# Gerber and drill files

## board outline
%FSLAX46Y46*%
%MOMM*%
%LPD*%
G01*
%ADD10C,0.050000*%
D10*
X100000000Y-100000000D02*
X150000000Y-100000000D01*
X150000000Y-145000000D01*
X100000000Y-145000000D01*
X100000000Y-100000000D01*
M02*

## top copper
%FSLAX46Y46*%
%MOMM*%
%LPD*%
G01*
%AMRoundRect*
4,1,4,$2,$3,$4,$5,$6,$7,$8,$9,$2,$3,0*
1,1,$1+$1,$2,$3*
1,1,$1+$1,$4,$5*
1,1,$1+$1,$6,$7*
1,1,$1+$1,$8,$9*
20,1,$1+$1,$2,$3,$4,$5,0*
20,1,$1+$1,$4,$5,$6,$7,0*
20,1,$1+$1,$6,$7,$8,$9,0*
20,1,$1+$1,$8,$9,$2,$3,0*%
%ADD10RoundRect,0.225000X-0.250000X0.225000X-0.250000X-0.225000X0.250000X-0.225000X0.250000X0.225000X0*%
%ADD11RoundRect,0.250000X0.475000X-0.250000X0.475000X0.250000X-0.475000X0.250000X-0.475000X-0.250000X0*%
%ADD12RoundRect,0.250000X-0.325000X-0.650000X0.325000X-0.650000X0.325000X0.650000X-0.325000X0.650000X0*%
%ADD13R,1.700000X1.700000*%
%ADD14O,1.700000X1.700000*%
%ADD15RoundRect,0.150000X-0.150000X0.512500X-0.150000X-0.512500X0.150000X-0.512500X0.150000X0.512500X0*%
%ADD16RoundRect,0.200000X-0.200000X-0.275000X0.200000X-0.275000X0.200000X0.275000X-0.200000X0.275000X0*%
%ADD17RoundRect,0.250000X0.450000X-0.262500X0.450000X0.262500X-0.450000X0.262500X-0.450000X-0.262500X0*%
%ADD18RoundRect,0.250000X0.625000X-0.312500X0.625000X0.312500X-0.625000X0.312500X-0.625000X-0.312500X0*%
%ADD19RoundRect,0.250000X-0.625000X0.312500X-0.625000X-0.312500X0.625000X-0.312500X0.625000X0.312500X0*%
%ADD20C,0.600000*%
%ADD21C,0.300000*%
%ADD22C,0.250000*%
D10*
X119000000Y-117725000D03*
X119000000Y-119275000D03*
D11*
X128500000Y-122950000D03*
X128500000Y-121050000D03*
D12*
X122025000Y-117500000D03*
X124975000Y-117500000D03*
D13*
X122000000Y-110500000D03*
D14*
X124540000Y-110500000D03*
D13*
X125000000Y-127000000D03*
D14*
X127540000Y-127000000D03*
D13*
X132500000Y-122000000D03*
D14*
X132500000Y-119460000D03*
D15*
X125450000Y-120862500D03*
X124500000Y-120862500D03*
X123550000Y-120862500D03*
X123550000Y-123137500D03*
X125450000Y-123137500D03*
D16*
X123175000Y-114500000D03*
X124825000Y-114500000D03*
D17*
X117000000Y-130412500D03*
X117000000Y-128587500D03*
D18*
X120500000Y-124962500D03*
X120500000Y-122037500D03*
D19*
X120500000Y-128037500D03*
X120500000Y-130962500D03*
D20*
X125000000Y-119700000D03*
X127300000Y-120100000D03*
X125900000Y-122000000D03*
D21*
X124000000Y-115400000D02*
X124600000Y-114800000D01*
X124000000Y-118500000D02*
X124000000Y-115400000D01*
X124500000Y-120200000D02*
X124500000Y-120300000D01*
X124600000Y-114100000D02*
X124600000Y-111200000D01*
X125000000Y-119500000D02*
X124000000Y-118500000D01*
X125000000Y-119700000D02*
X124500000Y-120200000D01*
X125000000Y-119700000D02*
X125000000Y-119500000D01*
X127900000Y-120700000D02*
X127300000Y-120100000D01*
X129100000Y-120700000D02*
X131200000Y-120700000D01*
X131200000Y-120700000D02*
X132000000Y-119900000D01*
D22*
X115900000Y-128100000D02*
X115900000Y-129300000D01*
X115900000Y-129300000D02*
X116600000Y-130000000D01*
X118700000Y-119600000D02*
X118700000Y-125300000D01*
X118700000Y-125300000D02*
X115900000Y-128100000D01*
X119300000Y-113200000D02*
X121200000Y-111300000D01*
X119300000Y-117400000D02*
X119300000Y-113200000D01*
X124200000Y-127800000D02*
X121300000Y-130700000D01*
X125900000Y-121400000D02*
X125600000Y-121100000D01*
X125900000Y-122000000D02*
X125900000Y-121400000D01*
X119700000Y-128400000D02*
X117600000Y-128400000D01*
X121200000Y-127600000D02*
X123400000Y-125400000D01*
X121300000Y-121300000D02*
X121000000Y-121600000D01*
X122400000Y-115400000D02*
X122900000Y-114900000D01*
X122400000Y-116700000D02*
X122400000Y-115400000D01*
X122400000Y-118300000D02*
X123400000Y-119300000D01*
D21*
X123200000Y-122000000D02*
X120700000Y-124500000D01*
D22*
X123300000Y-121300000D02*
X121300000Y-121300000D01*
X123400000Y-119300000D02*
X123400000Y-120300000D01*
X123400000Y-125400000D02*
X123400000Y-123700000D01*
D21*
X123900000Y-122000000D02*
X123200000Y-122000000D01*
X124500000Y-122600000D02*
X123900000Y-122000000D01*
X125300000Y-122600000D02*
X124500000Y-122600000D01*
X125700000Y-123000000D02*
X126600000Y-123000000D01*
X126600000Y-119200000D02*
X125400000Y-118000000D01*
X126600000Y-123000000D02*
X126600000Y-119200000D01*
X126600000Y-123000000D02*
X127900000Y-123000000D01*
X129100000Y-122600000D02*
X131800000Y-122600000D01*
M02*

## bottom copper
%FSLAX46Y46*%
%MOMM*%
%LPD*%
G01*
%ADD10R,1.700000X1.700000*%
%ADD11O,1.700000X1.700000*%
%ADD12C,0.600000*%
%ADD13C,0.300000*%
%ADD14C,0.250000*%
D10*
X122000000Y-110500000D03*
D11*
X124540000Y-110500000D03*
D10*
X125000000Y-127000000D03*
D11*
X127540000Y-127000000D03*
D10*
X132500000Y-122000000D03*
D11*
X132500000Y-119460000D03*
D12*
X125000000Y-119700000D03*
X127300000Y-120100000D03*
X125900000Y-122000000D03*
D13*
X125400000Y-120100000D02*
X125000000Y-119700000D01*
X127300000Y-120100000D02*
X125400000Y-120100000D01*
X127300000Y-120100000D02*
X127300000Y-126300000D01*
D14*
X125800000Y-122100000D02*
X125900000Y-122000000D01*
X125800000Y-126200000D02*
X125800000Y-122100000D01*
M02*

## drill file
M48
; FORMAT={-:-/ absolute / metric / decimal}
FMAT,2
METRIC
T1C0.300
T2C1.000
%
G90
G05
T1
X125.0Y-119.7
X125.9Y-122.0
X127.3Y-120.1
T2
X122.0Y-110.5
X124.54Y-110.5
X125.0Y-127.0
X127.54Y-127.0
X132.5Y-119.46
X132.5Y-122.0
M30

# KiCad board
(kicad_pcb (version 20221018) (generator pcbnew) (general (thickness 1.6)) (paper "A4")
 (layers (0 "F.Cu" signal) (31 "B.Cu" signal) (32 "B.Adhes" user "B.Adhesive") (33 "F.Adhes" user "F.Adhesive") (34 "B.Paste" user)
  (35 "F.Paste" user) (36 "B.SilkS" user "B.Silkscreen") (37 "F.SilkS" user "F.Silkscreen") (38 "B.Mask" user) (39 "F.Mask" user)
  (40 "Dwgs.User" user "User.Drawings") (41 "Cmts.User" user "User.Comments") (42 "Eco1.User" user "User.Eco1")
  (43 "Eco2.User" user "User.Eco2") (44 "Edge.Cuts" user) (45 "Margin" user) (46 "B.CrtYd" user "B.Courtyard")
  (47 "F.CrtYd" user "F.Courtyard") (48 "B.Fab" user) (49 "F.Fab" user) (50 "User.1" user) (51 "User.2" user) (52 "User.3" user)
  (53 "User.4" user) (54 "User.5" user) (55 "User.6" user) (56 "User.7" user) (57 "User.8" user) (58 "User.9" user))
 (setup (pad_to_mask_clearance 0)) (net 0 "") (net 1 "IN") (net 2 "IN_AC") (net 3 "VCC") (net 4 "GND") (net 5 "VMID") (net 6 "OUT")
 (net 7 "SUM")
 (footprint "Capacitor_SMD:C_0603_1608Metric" (layer "F.Cu") (at 119 118.5 -90)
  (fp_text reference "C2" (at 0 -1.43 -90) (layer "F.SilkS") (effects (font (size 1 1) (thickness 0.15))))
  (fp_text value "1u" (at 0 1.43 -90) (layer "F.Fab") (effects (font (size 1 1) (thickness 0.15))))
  (pad "1" smd roundrect (at -0.775 0 270) (size 0.9 0.95) (layers "F.Cu" "F.Paste" "F.Mask") (roundrect_rratio 0.25) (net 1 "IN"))
  (pad "2" smd roundrect (at 0.775 0 270) (size 0.9 0.95) (layers "F.Cu" "F.Paste" "F.Mask") (roundrect_rratio 0.25) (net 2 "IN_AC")))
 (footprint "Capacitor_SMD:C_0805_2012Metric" (layer "F.Cu") (at 128.5 122 90)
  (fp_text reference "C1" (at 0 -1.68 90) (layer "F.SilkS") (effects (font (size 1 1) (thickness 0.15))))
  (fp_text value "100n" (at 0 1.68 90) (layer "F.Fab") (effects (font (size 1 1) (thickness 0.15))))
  (pad "1" smd roundrect (at -0.95 0 90) (size 1 1.45) (layers "F.Cu" "F.Paste" "F.Mask") (roundrect_rratio 0.25) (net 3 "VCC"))
  (pad "2" smd roundrect (at 0.95 0 90) (size 1 1.45) (layers "F.Cu" "F.Paste" "F.Mask") (roundrect_rratio 0.25) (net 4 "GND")))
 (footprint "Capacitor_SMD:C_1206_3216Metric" (layer "F.Cu") (at 123.5 117.5)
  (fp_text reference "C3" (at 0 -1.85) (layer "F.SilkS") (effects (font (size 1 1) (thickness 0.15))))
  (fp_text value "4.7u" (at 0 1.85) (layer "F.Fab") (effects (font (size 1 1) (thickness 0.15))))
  (pad "1" smd roundrect (at -1.475 0) (size 1.15 1.8) (layers "F.Cu" "F.Paste" "F.Mask") (roundrect_rratio 0.217391) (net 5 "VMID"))
  (pad "2" smd roundrect (at 1.475 0) (size 1.15 1.8) (layers "F.Cu" "F.Paste" "F.Mask") (roundrect_rratio 0.217391) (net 3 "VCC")))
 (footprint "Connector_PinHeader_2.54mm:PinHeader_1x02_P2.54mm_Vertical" (layer "F.Cu") (at 122 110.5 90)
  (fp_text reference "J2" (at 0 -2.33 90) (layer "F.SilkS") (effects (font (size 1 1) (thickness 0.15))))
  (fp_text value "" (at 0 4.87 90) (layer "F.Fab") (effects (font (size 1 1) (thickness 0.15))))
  (pad "1" thru_hole rect (at 0 0 90) (size 1.7 1.7) (drill 1) (layers "*.Cu" "*.Mask") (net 1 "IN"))
  (pad "2" thru_hole oval (at 0 2.54 90) (size 1.7 1.7) (drill 1) (layers "*.Cu" "*.Mask") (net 4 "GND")))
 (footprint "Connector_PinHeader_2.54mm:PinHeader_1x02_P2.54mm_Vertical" (layer "F.Cu") (at 125 127 90)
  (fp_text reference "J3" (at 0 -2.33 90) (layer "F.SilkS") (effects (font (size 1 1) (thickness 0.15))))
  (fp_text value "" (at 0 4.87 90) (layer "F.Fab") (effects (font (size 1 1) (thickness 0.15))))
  (pad "1" thru_hole rect (at 0 0 90) (size 1.7 1.7) (drill 1) (layers "*.Cu" "*.Mask") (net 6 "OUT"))
  (pad "2" thru_hole oval (at 0 2.54 90) (size 1.7 1.7) (drill 1) (layers "*.Cu" "*.Mask") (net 4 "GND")))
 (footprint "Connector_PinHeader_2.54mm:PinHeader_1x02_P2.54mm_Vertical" (layer "F.Cu") (at 132.5 122 180)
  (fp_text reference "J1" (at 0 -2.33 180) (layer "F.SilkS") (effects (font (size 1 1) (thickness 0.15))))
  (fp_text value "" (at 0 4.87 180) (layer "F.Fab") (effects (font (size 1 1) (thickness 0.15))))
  (pad "1" thru_hole rect (at 0 0 180) (size 1.7 1.7) (drill 1) (layers "*.Cu" "*.Mask") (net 3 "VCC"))
  (pad "2" thru_hole oval (at 0 2.54 180) (size 1.7 1.7) (drill 1) (layers "*.Cu" "*.Mask") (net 4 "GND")))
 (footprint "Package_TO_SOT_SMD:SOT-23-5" (layer "F.Cu") (at 124.5 122 -90)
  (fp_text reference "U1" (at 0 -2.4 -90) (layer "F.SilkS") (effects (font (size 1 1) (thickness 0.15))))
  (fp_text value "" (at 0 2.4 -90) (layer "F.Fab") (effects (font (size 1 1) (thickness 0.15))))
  (pad "1" smd roundrect (at -1.1375 -0.95 270) (size 1.325 0.6) (layers "F.Cu" "F.Paste" "F.Mask") (roundrect_rratio 0.25) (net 6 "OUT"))
  (pad "2" smd roundrect (at -1.1375 0 270) (size 1.325 0.6) (layers "F.Cu" "F.Paste" "F.Mask") (roundrect_rratio 0.25) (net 4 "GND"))
  (pad "3" smd roundrect (at -1.1375 0.95 270) (size 1.325 0.6) (layers "F.Cu" "F.Paste" "F.Mask") (roundrect_rratio 0.25) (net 5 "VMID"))
  (pad "4" smd roundrect (at 1.1375 0.95 270) (size 1.325 0.6) (layers "F.Cu" "F.Paste" "F.Mask") (roundrect_rratio 0.25) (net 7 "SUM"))
  (pad "5" smd roundrect (at 1.1375 -0.95 270) (size 1.325 0.6) (layers "F.Cu" "F.Paste" "F.Mask") (roundrect_rratio 0.25) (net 3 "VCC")))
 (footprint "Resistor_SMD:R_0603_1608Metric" (layer "F.Cu") (at 124 114.5)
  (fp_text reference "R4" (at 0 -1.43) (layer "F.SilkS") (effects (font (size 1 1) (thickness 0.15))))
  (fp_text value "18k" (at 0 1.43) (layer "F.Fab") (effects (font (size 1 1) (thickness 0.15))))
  (pad "1" smd roundrect (at -0.825 0) (size 0.8 0.95) (layers "F.Cu" "F.Paste" "F.Mask") (roundrect_rratio 0.25) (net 5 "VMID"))
  (pad "2" smd roundrect (at 0.825 0) (size 0.8 0.95) (layers "F.Cu" "F.Paste" "F.Mask") (roundrect_rratio 0.25) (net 4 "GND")))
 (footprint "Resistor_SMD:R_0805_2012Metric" (layer "F.Cu") (at 117 129.5 90)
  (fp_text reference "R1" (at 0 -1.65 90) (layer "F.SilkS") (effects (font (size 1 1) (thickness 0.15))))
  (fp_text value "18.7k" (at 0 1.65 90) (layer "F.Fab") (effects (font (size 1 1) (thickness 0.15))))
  (pad "1" smd roundrect (at -0.9125 0 90) (size 1.025 1.4) (layers "F.Cu" "F.Paste" "F.Mask") (roundrect_rratio 0.243902) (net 2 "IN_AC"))
  (pad "2" smd roundrect (at 0.9125 0 90) (size 1.025 1.4) (layers "F.Cu" "F.Paste" "F.Mask") (roundrect_rratio 0.243902) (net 7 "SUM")))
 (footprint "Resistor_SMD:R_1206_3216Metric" (layer "F.Cu") (at 120.5 123.5 90)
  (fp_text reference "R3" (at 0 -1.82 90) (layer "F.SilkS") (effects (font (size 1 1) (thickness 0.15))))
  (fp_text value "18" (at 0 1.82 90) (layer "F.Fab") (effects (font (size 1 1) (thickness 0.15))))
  (pad "1" smd roundrect (at -1.4625 0 90) (size 1.125 1.75) (layers "F.Cu" "F.Paste" "F.Mask") (roundrect_rratio 0.222222) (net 3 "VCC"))
  (pad "2" smd roundrect (at 1.4625 0 90) (size 1.125 1.75) (layers "F.Cu" "F.Paste" "F.Mask") (roundrect_rratio 0.222222) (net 5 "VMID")))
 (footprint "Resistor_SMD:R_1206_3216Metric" (layer "F.Cu") (at 120.5 129.5 -90)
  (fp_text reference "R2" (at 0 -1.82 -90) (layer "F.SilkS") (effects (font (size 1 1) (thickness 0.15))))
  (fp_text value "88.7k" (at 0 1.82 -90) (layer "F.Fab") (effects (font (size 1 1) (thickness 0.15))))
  (pad "1" smd roundrect (at -1.4625 0 270) (size 1.125 1.75) (layers "F.Cu" "F.Paste" "F.Mask") (roundrect_rratio 0.222222) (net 7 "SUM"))
  (pad "2" smd roundrect (at 1.4625 0 270) (size 1.125 1.75) (layers "F.Cu" "F.Paste" "F.Mask") (roundrect_rratio 0.222222) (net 6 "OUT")))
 (gr_rect (start 100 100) (end 150 145) (stroke (width 0.05) (type default)) (fill none) (layer "Edge.Cuts"))
 (segment (start 124 115.4) (end 124.6 114.8) (width 0.3) (layer "F.Cu") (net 4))
 (segment (start 124 118.5) (end 124 115.4) (width 0.3) (layer "F.Cu") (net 4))
 (segment (start 124.5 120.2) (end 124.5 120.3) (width 0.3) (layer "F.Cu") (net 4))
 (segment (start 124.6 114.1) (end 124.6 111.2) (width 0.3) (layer "F.Cu") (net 4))
 (segment (start 125 119.5) (end 124 118.5) (width 0.3) (layer "F.Cu") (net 4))
 (segment (start 125 119.7) (end 124.5 120.2) (width 0.3) (layer "F.Cu") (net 4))
 (segment (start 125 119.7) (end 125 119.5) (width 0.3) (layer "F.Cu") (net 4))
 (segment (start 127.9 120.7) (end 127.3 120.1) (width 0.3) (layer "F.Cu") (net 4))
 (segment (start 129.1 120.7) (end 131.2 120.7) (width 0.3) (layer "F.Cu") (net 4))
 (segment (start 131.2 120.7) (end 132 119.9) (width 0.3) (layer "F.Cu") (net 4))
 (via (at 125 119.7) (size 0.6) (drill 0.3) (layers "F.Cu" "B.Cu") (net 4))
 (via (at 127.3 120.1) (size 0.6) (drill 0.3) (layers "F.Cu" "B.Cu") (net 4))
 (segment (start 115.9 128.1) (end 115.9 129.3) (width 0.25) (layer "F.Cu") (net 2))
 (segment (start 115.9 129.3) (end 116.6 130) (width 0.25) (layer "F.Cu") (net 2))
 (segment (start 118.7 119.6) (end 118.7 125.3) (width 0.25) (layer "F.Cu") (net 2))
 (segment (start 118.7 125.3) (end 115.9 128.1) (width 0.25) (layer "F.Cu") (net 2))
 (segment (start 119.3 113.2) (end 121.2 111.3) (width 0.25) (layer "F.Cu") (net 1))
 (segment (start 119.3 117.4) (end 119.3 113.2) (width 0.25) (layer "F.Cu") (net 1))
 (segment (start 124.2 127.8) (end 121.3 130.7) (width 0.25) (layer "F.Cu") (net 6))
 (segment (start 125.4 120.1) (end 125 119.7) (width 0.3) (layer "B.Cu") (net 4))
 (segment (start 125.9 121.4) (end 125.6 121.1) (width 0.25) (layer "F.Cu") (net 6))
 (segment (start 125.9 122) (end 125.9 121.4) (width 0.25) (layer "F.Cu") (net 6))
 (segment (start 127.3 120.1) (end 125.4 120.1) (width 0.3) (layer "B.Cu") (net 4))
 (segment (start 127.3 120.1) (end 127.3 126.3) (width 0.3) (layer "B.Cu") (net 4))
 (via (at 125.9 122) (size 0.6) (drill 0.3) (layers "F.Cu" "B.Cu") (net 6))
 (segment (start 119.7 128.4) (end 117.6 128.4) (width 0.25) (layer "F.Cu") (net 7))
 (segment (start 121.2 127.6) (end 123.4 125.4) (width 0.25) (layer "F.Cu") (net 7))
 (segment (start 121.3 121.3) (end 121 121.6) (width 0.25) (layer "F.Cu") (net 5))
 (segment (start 122.4 115.4) (end 122.9 114.9) (width 0.25) (layer "F.Cu") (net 5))
 (segment (start 122.4 116.7) (end 122.4 115.4) (width 0.25) (layer "F.Cu") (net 5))
 (segment (start 122.4 118.3) (end 123.4 119.3) (width 0.25) (layer "F.Cu") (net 5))
 (segment (start 123.2 122) (end 120.7 124.5) (width 0.3) (layer "F.Cu") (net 3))
 (segment (start 123.3 121.3) (end 121.3 121.3) (width 0.25) (layer "F.Cu") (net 5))
 (segment (start 123.4 119.3) (end 123.4 120.3) (width 0.25) (layer "F.Cu") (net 5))
 (segment (start 123.4 125.4) (end 123.4 123.7) (width 0.25) (layer "F.Cu") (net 7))
 (segment (start 123.9 122) (end 123.2 122) (width 0.3) (layer "F.Cu") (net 3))
 (segment (start 124.5 122.6) (end 123.9 122) (width 0.3) (layer "F.Cu") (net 3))
 (segment (start 125.3 122.6) (end 124.5 122.6) (width 0.3) (layer "F.Cu") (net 3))
 (segment (start 125.7 123) (end 126.6 123) (width 0.3) (layer "F.Cu") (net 3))
 (segment (start 125.8 122.1) (end 125.9 122) (width 0.25) (layer "B.Cu") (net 6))
 (segment (start 125.8 126.2) (end 125.8 122.1) (width 0.25) (layer "B.Cu") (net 6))
 (segment (start 126.6 119.2) (end 125.4 118) (width 0.3) (layer "F.Cu") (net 3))
 (segment (start 126.6 123) (end 126.6 119.2) (width 0.3) (layer "F.Cu") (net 3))
 (segment (start 126.6 123) (end 127.9 123) (width 0.3) (layer "F.Cu") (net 3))
 (segment (start 129.1 122.6) (end 131.8 122.6) (width 0.3) (layer "F.Cu") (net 3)))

